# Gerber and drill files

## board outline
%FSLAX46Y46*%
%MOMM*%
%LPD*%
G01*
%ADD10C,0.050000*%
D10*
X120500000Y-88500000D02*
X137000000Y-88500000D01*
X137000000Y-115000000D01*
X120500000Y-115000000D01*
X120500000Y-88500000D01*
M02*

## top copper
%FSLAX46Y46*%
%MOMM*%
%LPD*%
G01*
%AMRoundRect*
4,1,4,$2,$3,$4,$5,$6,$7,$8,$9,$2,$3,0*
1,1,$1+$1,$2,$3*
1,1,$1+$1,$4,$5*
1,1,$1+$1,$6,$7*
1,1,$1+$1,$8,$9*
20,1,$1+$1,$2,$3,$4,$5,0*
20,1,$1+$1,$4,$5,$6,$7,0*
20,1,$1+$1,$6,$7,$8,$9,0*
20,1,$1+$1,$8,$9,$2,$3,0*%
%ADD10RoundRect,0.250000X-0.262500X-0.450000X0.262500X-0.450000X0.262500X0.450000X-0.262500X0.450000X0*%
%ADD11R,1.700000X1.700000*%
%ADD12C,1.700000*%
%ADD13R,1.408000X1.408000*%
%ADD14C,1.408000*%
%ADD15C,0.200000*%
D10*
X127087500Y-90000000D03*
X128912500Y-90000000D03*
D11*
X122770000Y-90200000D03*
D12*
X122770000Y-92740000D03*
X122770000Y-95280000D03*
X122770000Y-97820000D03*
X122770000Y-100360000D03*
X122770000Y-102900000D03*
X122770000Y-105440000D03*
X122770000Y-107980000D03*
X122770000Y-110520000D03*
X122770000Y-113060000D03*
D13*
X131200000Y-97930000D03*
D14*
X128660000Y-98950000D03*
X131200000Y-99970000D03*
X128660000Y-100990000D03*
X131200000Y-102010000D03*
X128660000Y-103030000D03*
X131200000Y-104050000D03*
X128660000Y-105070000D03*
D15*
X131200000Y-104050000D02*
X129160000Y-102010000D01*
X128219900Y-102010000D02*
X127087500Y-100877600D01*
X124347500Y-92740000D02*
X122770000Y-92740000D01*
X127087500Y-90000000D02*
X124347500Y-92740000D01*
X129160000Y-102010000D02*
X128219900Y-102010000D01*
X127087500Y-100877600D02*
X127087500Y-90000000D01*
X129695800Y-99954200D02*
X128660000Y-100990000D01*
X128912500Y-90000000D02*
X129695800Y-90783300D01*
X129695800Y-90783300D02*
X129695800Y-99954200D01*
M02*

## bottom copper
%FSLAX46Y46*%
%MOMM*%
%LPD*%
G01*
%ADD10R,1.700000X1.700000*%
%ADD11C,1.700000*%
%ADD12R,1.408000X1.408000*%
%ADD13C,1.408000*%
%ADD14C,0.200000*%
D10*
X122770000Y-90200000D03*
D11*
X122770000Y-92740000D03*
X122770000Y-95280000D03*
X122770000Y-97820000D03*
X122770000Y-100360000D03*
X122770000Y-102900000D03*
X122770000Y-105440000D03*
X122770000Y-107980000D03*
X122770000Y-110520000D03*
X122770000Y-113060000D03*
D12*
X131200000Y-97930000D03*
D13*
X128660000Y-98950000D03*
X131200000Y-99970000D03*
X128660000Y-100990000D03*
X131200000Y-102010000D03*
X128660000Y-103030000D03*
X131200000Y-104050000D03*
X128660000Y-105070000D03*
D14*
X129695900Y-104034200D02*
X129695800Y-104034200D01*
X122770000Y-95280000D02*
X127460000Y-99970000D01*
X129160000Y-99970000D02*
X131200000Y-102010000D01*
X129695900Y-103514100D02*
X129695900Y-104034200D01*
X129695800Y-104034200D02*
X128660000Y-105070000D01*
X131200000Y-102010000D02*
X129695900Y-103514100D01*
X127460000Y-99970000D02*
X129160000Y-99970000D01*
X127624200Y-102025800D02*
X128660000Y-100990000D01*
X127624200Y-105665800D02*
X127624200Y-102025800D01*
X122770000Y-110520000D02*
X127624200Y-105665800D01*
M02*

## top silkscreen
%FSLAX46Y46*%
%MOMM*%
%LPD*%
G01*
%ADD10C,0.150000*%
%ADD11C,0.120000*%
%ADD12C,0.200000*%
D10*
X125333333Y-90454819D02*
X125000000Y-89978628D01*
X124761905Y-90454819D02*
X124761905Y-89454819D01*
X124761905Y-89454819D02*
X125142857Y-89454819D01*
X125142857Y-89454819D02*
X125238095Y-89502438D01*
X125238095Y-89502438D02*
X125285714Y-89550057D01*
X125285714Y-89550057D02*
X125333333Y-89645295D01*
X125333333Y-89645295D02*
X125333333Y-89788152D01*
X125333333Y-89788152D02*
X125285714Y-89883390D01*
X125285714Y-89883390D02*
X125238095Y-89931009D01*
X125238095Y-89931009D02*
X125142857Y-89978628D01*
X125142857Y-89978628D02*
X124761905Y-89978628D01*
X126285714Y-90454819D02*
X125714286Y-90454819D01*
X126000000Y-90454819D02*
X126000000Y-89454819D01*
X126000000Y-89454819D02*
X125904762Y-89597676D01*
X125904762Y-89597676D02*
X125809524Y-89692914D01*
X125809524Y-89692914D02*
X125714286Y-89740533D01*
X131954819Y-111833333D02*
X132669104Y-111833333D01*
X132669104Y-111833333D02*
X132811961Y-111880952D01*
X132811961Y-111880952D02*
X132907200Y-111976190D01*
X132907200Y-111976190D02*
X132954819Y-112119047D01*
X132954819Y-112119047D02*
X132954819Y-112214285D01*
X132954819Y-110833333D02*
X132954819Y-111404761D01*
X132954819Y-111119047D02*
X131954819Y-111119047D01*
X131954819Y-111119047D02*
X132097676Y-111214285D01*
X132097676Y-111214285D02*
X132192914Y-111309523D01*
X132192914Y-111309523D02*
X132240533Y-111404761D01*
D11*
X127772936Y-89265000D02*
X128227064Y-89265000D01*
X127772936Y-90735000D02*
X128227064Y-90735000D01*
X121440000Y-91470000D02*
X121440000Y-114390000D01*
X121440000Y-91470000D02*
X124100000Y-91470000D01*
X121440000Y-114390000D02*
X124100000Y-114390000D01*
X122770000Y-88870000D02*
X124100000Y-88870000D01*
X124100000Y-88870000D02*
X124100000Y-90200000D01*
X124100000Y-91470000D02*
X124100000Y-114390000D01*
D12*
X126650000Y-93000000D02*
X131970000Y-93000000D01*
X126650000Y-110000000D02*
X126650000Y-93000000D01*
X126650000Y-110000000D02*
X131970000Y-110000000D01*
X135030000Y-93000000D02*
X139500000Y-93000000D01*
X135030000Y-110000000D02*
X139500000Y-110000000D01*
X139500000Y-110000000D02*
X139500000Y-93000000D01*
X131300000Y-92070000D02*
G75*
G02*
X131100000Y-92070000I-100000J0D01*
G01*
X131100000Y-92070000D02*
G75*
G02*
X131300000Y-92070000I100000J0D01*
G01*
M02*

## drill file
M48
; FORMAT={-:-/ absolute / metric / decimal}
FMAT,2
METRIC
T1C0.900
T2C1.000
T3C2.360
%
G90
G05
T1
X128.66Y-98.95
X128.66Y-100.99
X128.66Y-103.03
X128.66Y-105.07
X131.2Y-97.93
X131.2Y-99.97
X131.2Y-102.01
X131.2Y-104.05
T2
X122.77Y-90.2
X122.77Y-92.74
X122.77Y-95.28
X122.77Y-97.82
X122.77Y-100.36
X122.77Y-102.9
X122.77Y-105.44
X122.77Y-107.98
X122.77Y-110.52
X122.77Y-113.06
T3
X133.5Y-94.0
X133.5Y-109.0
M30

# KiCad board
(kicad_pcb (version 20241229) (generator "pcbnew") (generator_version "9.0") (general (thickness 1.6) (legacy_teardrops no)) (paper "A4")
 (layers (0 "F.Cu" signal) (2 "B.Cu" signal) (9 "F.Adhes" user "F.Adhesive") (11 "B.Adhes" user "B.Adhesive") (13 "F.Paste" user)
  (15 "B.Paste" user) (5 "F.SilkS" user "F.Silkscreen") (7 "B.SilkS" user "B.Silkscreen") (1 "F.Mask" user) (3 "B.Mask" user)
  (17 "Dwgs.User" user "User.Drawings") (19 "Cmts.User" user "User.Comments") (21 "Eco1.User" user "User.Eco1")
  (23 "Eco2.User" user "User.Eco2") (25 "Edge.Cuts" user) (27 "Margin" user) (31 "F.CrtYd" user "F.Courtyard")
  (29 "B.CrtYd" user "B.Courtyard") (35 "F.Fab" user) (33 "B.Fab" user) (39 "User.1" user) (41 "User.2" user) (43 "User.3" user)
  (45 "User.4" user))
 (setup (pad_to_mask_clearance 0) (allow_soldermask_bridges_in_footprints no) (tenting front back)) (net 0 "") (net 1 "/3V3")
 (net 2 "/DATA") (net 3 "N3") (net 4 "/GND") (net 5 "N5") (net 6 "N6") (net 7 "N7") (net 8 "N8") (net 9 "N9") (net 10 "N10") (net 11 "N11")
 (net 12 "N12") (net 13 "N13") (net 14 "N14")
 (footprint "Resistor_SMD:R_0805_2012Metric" (layer "F.Cu") (at 128 90)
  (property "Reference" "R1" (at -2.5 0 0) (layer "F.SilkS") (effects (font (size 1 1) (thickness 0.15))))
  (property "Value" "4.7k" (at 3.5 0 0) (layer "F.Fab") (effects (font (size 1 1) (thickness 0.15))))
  (fp_line (start -0.227064 -0.735) (end 0.227064 -0.735) (stroke (width 0.12) (type solid)) (layer "F.SilkS"))
  (fp_line (start -0.227064 0.735) (end 0.227064 0.735) (stroke (width 0.12) (type solid)) (layer "F.SilkS"))
  (pad "1" smd roundrect (at -0.9125 0) (size 1.025 1.4) (layers "F.Cu" "F.Mask" "F.Paste") (roundrect_rratio 0.243902) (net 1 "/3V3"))
  (pad "2" smd roundrect (at 0.9125 0) (size 1.025 1.4) (layers "F.Cu" "F.Mask" "F.Paste") (roundrect_rratio 0.243902) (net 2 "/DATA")))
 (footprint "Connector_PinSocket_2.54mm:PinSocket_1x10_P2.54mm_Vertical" (layer "F.Cu") (at 122.77 90.2)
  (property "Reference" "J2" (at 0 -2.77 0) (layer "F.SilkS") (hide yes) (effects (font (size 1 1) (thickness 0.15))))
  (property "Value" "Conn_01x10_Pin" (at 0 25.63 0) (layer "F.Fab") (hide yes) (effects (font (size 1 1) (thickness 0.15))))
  (fp_line (start -1.33 1.27) (end -1.33 24.19) (stroke (width 0.12) (type solid)) (layer "F.SilkS"))
  (fp_line (start -1.33 1.27) (end 1.33 1.27) (stroke (width 0.12) (type solid)) (layer "F.SilkS"))
  (fp_line (start -1.33 24.19) (end 1.33 24.19) (stroke (width 0.12) (type solid)) (layer "F.SilkS"))
  (fp_line (start 0 -1.33) (end 1.33 -1.33) (stroke (width 0.12) (type solid)) (layer "F.SilkS"))
  (fp_line (start 1.33 -1.33) (end 1.33 0) (stroke (width 0.12) (type solid)) (layer "F.SilkS"))
  (fp_line (start 1.33 1.27) (end 1.33 24.19) (stroke (width 0.12) (type solid)) (layer "F.SilkS"))
  (pad "1" thru_hole rect (at 0 0) (size 1.7 1.7) (drill 1) (layers "*.Cu" "*.Mask") (remove_unused_layers no) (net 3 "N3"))
  (pad "2" thru_hole circle (at 0 2.54) (size 1.7 1.7) (drill 1) (layers "*.Cu" "*.Mask") (remove_unused_layers no) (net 1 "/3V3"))
  (pad "3" thru_hole circle (at 0 5.08) (size 1.7 1.7) (drill 1) (layers "*.Cu" "*.Mask") (remove_unused_layers no) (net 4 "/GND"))
  (pad "4" thru_hole circle (at 0 7.62) (size 1.7 1.7) (drill 1) (layers "*.Cu" "*.Mask") (remove_unused_layers no) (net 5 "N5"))
  (pad "5" thru_hole circle (at 0 10.16) (size 1.7 1.7) (drill 1) (layers "*.Cu" "*.Mask") (remove_unused_layers no) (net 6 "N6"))
  (pad "6" thru_hole circle (at 0 12.7) (size 1.7 1.7) (drill 1) (layers "*.Cu" "*.Mask") (remove_unused_layers no) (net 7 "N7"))
  (pad "7" thru_hole circle (at 0 15.24) (size 1.7 1.7) (drill 1) (layers "*.Cu" "*.Mask") (remove_unused_layers no) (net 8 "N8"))
  (pad "8" thru_hole circle (at 0 17.78) (size 1.7 1.7) (drill 1) (layers "*.Cu" "*.Mask") (remove_unused_layers no) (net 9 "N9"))
  (pad "9" thru_hole circle (at 0 20.32) (size 1.7 1.7) (drill 1) (layers "*.Cu" "*.Mask") (remove_unused_layers no) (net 2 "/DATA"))
  (pad "10" thru_hole circle (at 0 22.86) (size 1.7 1.7) (drill 1) (layers "*.Cu" "*.Mask") (remove_unused_layers no) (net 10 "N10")))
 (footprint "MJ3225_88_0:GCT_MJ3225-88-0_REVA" (layer "F.Cu") (at 133.075 101.5 90)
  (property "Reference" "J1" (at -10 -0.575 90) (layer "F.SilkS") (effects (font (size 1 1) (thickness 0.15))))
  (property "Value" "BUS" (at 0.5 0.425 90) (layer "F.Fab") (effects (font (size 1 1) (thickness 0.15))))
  (fp_line (start 8.5 -6.425) (end 8.5 -1.105) (stroke (width 0.2) (type solid)) (layer "F.SilkS"))
  (fp_line (start -8.5 -6.425) (end 8.5 -6.425) (stroke (width 0.2) (type solid)) (layer "F.SilkS"))
  (fp_line (start -8.5 -6.425) (end -8.5 -1.105) (stroke (width 0.2) (type solid)) (layer "F.SilkS"))
  (fp_line (start 8.5 1.955) (end 8.5 6.425) (stroke (width 0.2) (type solid)) (layer "F.SilkS"))
  (fp_line (start -8.5 1.955) (end -8.5 6.425) (stroke (width 0.2) (type solid)) (layer "F.SilkS"))
  (fp_line (start -8.5 6.425) (end 8.5 6.425) (stroke (width 0.2) (type solid)) (layer "F.SilkS"))
  (fp_circle (center 9.43 -1.875) (end 9.53 -1.875) (stroke (width 0.2) (type solid)) (fill no) (layer "F.SilkS"))
  (pad "" np_thru_hole circle (at -7.5 0.425 90) (size 2.36 2.36) (drill 2.36) (layers "*.Cu" "*.Mask"))
  (pad "" np_thru_hole circle (at 7.5 0.425 90) (size 2.36 2.36) (drill 2.36) (layers "*.Cu" "*.Mask"))
  (pad "1" thru_hole rect (at 3.57 -1.875 90) (size 1.408 1.408) (drill 0.9) (layers "*.Cu" "*.Mask") (remove_unused_layers no)
   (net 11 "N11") (solder_mask_margin 0.102))
  (pad "2" thru_hole circle (at 2.55 -4.415 90) (size 1.408 1.408) (drill 0.9) (layers "*.Cu" "*.Mask") (remove_unused_layers no)
   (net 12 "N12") (solder_mask_margin 0.102))
  (pad "3" thru_hole circle (at 1.53 -1.875 90) (size 1.408 1.408) (drill 0.9) (layers "*.Cu" "*.Mask") (remove_unused_layers no)
   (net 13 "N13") (solder_mask_margin 0.102))
  (pad "4" thru_hole circle (at 0.51 -4.415 90) (size 1.408 1.408) (drill 0.9) (layers "*.Cu" "*.Mask") (remove_unused_layers no)
   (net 2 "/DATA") (solder_mask_margin 0.102))
  (pad "5" thru_hole circle (at -0.51 -1.875 90) (size 1.408 1.408) (drill 0.9) (layers "*.Cu" "*.Mask") (remove_unused_layers no)
   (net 4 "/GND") (solder_mask_margin 0.102))
  (pad "6" thru_hole circle (at -1.53 -4.415 90) (size 1.408 1.408) (drill 0.9) (layers "*.Cu" "*.Mask") (remove_unused_layers no)
   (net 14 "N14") (solder_mask_margin 0.102))
  (pad "7" thru_hole circle (at -2.55 -1.875 90) (size 1.408 1.408) (drill 0.9) (layers "*.Cu" "*.Mask") (remove_unused_layers no)
   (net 1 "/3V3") (solder_mask_margin 0.102))
  (pad "8" thru_hole circle (at -3.57 -4.415 90) (size 1.408 1.408) (drill 0.9) (layers "*.Cu" "*.Mask") (remove_unused_layers no)
   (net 4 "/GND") (solder_mask_margin 0.102)))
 (gr_rect (start 120.5 88.5) (end 137 115) (stroke (width 0.05) (type default)) (fill no) (layer "Edge.Cuts"))
 (segment (start 129.6959 104.0342) (end 129.6958 104.0342) (width 0.2) (layer "B.Cu") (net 4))
 (segment (start 122.77 95.28) (end 127.46 99.97) (width 0.2) (layer "B.Cu") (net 4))
 (segment (start 129.16 99.97) (end 131.2 102.01) (width 0.2) (layer "B.Cu") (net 4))
 (segment (start 129.6959 103.5141) (end 129.6959 104.0342) (width 0.2) (layer "B.Cu") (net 4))
 (segment (start 129.6958 104.0342) (end 128.66 105.07) (width 0.2) (layer "B.Cu") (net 4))
 (segment (start 131.2 102.01) (end 129.6959 103.5141) (width 0.2) (layer "B.Cu") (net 4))
 (segment (start 127.46 99.97) (end 129.16 99.97) (width 0.2) (layer "B.Cu") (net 4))
 (segment (start 131.2 104.05) (end 129.16 102.01) (width 0.2) (layer "F.Cu") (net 1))
 (segment (start 128.2199 102.01) (end 127.0875 100.8776) (width 0.2) (layer "F.Cu") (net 1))
 (segment (start 124.3475 92.74) (end 122.77 92.74) (width 0.2) (layer "F.Cu") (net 1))
 (segment (start 127.0875 90) (end 124.3475 92.74) (width 0.2) (layer "F.Cu") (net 1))
 (segment (start 129.16 102.01) (end 128.2199 102.01) (width 0.2) (layer "F.Cu") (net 1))
 (segment (start 127.0875 100.8776) (end 127.0875 90) (width 0.2) (layer "F.Cu") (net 1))
 (segment (start 129.6958 99.9542) (end 128.66 100.99) (width 0.2) (layer "F.Cu") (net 2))
 (segment (start 128.9125 90) (end 129.6958 90.7833) (width 0.2) (layer "F.Cu") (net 2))
 (segment (start 129.6958 90.7833) (end 129.6958 99.9542) (width 0.2) (layer "F.Cu") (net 2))
 (segment (start 127.6242 102.0258) (end 128.66 100.99) (width 0.2) (layer "B.Cu") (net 2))
 (segment (start 127.6242 105.6658) (end 127.6242 102.0258) (width 0.2) (layer "B.Cu") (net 2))
 (segment (start 122.77 110.52) (end 127.6242 105.6658) (width 0.2) (layer "B.Cu") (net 2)))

